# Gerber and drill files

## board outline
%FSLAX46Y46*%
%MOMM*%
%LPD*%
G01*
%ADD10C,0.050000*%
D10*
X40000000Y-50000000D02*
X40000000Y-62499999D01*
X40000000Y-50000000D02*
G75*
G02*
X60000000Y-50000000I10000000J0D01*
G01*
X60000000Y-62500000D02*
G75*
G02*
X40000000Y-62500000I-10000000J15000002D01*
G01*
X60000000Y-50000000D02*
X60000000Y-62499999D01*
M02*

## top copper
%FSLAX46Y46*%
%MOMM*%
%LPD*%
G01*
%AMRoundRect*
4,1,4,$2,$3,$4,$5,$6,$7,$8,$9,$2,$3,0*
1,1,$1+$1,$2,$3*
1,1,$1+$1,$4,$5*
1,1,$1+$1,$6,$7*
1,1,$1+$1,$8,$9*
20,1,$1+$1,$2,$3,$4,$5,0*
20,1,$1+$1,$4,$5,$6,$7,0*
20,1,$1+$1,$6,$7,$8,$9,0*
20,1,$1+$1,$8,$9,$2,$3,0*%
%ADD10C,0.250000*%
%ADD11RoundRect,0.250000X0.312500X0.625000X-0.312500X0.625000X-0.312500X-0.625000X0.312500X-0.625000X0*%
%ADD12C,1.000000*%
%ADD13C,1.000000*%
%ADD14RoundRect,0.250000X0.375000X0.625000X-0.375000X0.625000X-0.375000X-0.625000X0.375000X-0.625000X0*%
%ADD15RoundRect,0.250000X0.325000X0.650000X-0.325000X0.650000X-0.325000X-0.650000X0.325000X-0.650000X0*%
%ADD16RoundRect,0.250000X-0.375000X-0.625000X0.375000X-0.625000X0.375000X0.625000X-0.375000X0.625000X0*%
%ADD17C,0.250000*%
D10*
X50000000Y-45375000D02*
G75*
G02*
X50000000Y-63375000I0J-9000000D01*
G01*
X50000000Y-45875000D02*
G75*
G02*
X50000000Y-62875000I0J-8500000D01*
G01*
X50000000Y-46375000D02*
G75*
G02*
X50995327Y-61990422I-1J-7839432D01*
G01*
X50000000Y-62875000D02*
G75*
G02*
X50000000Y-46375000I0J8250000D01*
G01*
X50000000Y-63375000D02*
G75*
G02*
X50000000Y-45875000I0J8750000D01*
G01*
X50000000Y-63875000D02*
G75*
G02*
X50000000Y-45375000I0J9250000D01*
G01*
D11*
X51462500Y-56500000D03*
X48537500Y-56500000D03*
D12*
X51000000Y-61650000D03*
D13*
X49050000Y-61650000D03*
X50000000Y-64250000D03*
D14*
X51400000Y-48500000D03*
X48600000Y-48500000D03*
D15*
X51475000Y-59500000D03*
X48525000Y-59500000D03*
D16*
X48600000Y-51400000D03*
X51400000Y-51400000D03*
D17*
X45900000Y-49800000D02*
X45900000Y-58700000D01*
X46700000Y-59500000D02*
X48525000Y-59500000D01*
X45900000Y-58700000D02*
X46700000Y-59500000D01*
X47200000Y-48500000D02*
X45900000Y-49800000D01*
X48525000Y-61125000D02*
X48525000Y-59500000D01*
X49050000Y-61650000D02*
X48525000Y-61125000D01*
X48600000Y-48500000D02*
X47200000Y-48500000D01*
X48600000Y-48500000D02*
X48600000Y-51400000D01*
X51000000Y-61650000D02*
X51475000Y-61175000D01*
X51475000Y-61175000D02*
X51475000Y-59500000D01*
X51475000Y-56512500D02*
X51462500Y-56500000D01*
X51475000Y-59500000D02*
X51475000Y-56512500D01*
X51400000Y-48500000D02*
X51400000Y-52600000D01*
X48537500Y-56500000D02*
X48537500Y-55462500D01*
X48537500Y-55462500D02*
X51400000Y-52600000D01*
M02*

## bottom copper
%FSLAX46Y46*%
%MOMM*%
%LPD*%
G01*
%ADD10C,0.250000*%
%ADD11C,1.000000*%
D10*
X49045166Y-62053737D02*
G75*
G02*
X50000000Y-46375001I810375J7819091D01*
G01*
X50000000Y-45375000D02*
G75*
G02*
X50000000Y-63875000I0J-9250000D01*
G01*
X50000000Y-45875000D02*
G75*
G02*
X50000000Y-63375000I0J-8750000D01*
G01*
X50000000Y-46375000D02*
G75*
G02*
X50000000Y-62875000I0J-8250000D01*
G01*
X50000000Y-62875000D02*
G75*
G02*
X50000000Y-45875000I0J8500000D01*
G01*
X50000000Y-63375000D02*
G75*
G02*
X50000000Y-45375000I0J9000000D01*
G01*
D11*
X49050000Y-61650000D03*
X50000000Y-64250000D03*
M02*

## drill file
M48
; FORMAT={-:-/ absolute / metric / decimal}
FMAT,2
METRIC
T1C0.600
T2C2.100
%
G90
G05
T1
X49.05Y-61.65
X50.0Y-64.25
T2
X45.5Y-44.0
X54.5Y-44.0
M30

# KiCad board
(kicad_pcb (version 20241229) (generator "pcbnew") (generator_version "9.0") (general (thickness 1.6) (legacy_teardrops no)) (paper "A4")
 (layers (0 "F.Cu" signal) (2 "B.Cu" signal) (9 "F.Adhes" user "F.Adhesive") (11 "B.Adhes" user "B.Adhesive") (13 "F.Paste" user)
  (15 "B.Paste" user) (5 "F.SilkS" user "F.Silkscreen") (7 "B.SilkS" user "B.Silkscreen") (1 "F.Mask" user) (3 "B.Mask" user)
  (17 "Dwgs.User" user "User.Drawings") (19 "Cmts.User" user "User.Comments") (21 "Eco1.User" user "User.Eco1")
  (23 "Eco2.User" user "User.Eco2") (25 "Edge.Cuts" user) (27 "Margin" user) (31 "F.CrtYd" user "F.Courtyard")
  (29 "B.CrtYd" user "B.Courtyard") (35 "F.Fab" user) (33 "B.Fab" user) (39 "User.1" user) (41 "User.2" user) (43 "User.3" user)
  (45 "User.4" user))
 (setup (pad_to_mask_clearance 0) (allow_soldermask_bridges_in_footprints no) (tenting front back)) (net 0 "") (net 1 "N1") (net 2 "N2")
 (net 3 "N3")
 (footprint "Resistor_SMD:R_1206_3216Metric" (layer "F.Cu") (at 50 56.5 180)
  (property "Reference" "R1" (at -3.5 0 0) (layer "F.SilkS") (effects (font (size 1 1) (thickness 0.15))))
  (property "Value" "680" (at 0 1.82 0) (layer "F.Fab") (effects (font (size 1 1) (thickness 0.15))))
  (pad "1" smd roundrect (at -1.4625 0 180) (size 1.125 1.75) (layers "F.Cu" "F.Mask" "F.Paste") (roundrect_rratio 0.222222) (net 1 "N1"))
  (pad "2" smd roundrect (at 1.4625 0 180) (size 1.125 1.75) (layers "F.Cu" "F.Mask" "F.Paste") (roundrect_rratio 0.222222) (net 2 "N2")))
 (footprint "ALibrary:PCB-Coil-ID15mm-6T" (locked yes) (layer "F.Cu") (at 50 54 -90)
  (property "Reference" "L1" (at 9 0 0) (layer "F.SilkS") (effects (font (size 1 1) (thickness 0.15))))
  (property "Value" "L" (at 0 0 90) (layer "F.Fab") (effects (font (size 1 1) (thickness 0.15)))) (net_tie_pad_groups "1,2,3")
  (fp_arc (start -8.625 0) (mid 0.375 -9) (end 9.375 0) (stroke (width 0.25) (type default)) (layer "F.Cu"))
  (fp_arc (start -8.125 0) (mid 0.375 -8.5) (end 8.875 0) (stroke (width 0.25) (type default)) (layer "F.Cu"))
  (fp_arc (start -7.625 0) (mid -0.284241 -7.823555) (end 7.990422 -0.995327) (stroke (width 0.25) (type default)) (layer "F.Cu"))
  (fp_arc (start 8.875 0) (mid 0.625 8.25) (end -7.625 0) (stroke (width 0.25) (type default)) (layer "F.Cu"))
  (fp_arc (start 9.375 0) (mid 0.625 8.75) (end -8.125 0) (stroke (width 0.25) (type default)) (layer "F.Cu"))
  (fp_arc (start 9.875 0) (mid 0.625 9.25) (end -8.625 0) (stroke (width 0.25) (type default)) (layer "F.Cu"))
  (fp_arc (start 8.053737 0.954834) (mid -0.243201 7.990895) (end -7.625 0) (stroke (width 0.25) (type default)) (layer "B.Cu"))
  (fp_arc (start -8.625 0) (mid 0.625 -9.25) (end 9.875 0) (stroke (width 0.25) (type default)) (layer "B.Cu"))
  (fp_arc (start -8.125 0) (mid 0.625 -8.75) (end 9.375 0) (stroke (width 0.25) (type default)) (layer "B.Cu"))
  (fp_arc (start -7.625 0) (mid 0.625 -8.25) (end 8.875 0) (stroke (width 0.25) (type default)) (layer "B.Cu"))
  (fp_arc (start 8.875 0) (mid 0.375 8.5) (end -8.125 0) (stroke (width 0.25) (type default)) (layer "B.Cu"))
  (fp_arc (start 9.375 0) (mid 0.375 9) (end -8.625 0) (stroke (width 0.25) (type default)) (layer "B.Cu"))
  (pad "1" smd circle (at 7.65 -1 270) (size 1 1) (layers "F.Cu" "F.Mask" "F.Paste") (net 1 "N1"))
  (pad "2" thru_hole circle (at 7.65 0.95 270) (size 1 1) (drill 0.6) (layers "*.Cu") (remove_unused_layers no) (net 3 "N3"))
  (pad "3" thru_hole circle (at 10.25 0 270) (size 1 1) (drill 0.6) (layers "*.Cu") (remove_unused_layers no)))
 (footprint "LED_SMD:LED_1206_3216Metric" (layer "F.Cu") (at 50 48.5 180)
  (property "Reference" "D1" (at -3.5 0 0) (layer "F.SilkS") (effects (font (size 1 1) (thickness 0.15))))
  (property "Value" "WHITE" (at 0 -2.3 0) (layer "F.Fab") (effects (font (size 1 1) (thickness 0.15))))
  (pad "1" smd roundrect (at -1.4 0 180) (size 1.25 1.75) (layers "F.Cu" "F.Mask" "F.Paste") (roundrect_rratio 0.2) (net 2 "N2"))
  (pad "2" smd roundrect (at 1.4 0 180) (size 1.25 1.75) (layers "F.Cu" "F.Mask" "F.Paste") (roundrect_rratio 0.2) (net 3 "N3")))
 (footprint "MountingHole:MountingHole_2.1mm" (layer "F.Cu") (at 54.5 44)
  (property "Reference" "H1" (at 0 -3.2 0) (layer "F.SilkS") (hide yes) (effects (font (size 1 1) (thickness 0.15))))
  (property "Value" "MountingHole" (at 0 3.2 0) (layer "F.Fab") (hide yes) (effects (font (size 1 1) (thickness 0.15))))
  (pad "" np_thru_hole circle (at 0 0) (size 2.1 2.1) (drill 2.1) (layers "*.Cu" "*.Mask")))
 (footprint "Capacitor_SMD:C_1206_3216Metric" (layer "F.Cu") (at 50 59.5 180)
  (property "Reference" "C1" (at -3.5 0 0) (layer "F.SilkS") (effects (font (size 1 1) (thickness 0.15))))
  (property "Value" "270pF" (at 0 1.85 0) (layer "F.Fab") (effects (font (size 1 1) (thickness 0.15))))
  (pad "1" smd roundrect (at -1.475 0 180) (size 1.15 1.8) (layers "F.Cu" "F.Mask" "F.Paste") (roundrect_rratio 0.217391) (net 1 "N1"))
  (pad "2" smd roundrect (at 1.475 0 180) (size 1.15 1.8) (layers "F.Cu" "F.Mask" "F.Paste") (roundrect_rratio 0.217391) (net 3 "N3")))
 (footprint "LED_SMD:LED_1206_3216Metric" (layer "F.Cu") (at 50 51.4)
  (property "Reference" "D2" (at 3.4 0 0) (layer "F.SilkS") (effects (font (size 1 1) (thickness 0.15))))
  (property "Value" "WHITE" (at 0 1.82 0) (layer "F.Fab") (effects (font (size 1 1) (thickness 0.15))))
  (pad "1" smd roundrect (at -1.4 0) (size 1.25 1.75) (layers "F.Cu" "F.Mask" "F.Paste") (roundrect_rratio 0.2) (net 3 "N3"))
  (pad "2" smd roundrect (at 1.4 0) (size 1.25 1.75) (layers "F.Cu" "F.Mask" "F.Paste") (roundrect_rratio 0.2) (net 2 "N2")))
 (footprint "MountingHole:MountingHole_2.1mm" (layer "F.Cu") (at 45.5 44)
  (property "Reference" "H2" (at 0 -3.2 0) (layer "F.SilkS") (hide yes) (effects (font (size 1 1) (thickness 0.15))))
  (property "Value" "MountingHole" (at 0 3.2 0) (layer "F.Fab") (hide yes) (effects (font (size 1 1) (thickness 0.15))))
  (pad "" np_thru_hole circle (at 0 0) (size 2.1 2.1) (drill 2.1) (layers "*.Cu" "*.Mask")))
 (gr_line (start 40 50) (end 40 62.499999) (stroke (width 0.05) (type default)) (layer "Edge.Cuts"))
 (gr_arc (start 40 50) (mid 50 40) (end 60 50) (stroke (width 0.05) (type default)) (layer "Edge.Cuts"))
 (gr_arc (start 60 62.5) (mid 50 65.527756) (end 40 62.5) (stroke (width 0.05) (type default)) (layer "Edge.Cuts"))
 (gr_line (start 60 50) (end 60 62.499999) (stroke (width 0.05) (type default)) (layer "Edge.Cuts"))
 (segment (start 45.9 49.8) (end 45.9 58.7) (width 0.25) (layer "F.Cu") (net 3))
 (segment (start 46.7 59.5) (end 48.525 59.5) (width 0.25) (layer "F.Cu") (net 3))
 (segment (start 45.9 58.7) (end 46.7 59.5) (width 0.25) (layer "F.Cu") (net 3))
 (segment (start 47.2 48.5) (end 45.9 49.8) (width 0.25) (layer "F.Cu") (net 3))
 (segment (start 48.525 61.125) (end 48.525 59.5) (width 0.25) (layer "F.Cu") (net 3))
 (segment (start 49.05 61.65) (end 48.525 61.125) (width 0.25) (layer "F.Cu") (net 3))
 (segment (start 48.6 48.5) (end 47.2 48.5) (width 0.25) (layer "F.Cu") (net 3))
 (segment (start 48.6 48.5) (end 48.6 51.4) (width 0.25) (layer "F.Cu") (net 3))
 (segment (start 51 61.65) (end 51.475 61.175) (width 0.25) (layer "F.Cu") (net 1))
 (segment (start 51.475 61.175) (end 51.475 59.5) (width 0.25) (layer "F.Cu") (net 1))
 (segment (start 51.475 56.5125) (end 51.4625 56.5) (width 0.25) (layer "F.Cu") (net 1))
 (segment (start 51.475 59.5) (end 51.475 56.5125) (width 0.25) (layer "F.Cu") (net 1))
 (segment (start 51.4 48.5) (end 51.4 52.6) (width 0.25) (layer "F.Cu") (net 2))
 (segment (start 48.5375 56.5) (end 48.5375 55.4625) (width 0.25) (layer "F.Cu") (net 2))
 (segment (start 48.5375 55.4625) (end 51.4 52.6) (width 0.25) (layer "F.Cu") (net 2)))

